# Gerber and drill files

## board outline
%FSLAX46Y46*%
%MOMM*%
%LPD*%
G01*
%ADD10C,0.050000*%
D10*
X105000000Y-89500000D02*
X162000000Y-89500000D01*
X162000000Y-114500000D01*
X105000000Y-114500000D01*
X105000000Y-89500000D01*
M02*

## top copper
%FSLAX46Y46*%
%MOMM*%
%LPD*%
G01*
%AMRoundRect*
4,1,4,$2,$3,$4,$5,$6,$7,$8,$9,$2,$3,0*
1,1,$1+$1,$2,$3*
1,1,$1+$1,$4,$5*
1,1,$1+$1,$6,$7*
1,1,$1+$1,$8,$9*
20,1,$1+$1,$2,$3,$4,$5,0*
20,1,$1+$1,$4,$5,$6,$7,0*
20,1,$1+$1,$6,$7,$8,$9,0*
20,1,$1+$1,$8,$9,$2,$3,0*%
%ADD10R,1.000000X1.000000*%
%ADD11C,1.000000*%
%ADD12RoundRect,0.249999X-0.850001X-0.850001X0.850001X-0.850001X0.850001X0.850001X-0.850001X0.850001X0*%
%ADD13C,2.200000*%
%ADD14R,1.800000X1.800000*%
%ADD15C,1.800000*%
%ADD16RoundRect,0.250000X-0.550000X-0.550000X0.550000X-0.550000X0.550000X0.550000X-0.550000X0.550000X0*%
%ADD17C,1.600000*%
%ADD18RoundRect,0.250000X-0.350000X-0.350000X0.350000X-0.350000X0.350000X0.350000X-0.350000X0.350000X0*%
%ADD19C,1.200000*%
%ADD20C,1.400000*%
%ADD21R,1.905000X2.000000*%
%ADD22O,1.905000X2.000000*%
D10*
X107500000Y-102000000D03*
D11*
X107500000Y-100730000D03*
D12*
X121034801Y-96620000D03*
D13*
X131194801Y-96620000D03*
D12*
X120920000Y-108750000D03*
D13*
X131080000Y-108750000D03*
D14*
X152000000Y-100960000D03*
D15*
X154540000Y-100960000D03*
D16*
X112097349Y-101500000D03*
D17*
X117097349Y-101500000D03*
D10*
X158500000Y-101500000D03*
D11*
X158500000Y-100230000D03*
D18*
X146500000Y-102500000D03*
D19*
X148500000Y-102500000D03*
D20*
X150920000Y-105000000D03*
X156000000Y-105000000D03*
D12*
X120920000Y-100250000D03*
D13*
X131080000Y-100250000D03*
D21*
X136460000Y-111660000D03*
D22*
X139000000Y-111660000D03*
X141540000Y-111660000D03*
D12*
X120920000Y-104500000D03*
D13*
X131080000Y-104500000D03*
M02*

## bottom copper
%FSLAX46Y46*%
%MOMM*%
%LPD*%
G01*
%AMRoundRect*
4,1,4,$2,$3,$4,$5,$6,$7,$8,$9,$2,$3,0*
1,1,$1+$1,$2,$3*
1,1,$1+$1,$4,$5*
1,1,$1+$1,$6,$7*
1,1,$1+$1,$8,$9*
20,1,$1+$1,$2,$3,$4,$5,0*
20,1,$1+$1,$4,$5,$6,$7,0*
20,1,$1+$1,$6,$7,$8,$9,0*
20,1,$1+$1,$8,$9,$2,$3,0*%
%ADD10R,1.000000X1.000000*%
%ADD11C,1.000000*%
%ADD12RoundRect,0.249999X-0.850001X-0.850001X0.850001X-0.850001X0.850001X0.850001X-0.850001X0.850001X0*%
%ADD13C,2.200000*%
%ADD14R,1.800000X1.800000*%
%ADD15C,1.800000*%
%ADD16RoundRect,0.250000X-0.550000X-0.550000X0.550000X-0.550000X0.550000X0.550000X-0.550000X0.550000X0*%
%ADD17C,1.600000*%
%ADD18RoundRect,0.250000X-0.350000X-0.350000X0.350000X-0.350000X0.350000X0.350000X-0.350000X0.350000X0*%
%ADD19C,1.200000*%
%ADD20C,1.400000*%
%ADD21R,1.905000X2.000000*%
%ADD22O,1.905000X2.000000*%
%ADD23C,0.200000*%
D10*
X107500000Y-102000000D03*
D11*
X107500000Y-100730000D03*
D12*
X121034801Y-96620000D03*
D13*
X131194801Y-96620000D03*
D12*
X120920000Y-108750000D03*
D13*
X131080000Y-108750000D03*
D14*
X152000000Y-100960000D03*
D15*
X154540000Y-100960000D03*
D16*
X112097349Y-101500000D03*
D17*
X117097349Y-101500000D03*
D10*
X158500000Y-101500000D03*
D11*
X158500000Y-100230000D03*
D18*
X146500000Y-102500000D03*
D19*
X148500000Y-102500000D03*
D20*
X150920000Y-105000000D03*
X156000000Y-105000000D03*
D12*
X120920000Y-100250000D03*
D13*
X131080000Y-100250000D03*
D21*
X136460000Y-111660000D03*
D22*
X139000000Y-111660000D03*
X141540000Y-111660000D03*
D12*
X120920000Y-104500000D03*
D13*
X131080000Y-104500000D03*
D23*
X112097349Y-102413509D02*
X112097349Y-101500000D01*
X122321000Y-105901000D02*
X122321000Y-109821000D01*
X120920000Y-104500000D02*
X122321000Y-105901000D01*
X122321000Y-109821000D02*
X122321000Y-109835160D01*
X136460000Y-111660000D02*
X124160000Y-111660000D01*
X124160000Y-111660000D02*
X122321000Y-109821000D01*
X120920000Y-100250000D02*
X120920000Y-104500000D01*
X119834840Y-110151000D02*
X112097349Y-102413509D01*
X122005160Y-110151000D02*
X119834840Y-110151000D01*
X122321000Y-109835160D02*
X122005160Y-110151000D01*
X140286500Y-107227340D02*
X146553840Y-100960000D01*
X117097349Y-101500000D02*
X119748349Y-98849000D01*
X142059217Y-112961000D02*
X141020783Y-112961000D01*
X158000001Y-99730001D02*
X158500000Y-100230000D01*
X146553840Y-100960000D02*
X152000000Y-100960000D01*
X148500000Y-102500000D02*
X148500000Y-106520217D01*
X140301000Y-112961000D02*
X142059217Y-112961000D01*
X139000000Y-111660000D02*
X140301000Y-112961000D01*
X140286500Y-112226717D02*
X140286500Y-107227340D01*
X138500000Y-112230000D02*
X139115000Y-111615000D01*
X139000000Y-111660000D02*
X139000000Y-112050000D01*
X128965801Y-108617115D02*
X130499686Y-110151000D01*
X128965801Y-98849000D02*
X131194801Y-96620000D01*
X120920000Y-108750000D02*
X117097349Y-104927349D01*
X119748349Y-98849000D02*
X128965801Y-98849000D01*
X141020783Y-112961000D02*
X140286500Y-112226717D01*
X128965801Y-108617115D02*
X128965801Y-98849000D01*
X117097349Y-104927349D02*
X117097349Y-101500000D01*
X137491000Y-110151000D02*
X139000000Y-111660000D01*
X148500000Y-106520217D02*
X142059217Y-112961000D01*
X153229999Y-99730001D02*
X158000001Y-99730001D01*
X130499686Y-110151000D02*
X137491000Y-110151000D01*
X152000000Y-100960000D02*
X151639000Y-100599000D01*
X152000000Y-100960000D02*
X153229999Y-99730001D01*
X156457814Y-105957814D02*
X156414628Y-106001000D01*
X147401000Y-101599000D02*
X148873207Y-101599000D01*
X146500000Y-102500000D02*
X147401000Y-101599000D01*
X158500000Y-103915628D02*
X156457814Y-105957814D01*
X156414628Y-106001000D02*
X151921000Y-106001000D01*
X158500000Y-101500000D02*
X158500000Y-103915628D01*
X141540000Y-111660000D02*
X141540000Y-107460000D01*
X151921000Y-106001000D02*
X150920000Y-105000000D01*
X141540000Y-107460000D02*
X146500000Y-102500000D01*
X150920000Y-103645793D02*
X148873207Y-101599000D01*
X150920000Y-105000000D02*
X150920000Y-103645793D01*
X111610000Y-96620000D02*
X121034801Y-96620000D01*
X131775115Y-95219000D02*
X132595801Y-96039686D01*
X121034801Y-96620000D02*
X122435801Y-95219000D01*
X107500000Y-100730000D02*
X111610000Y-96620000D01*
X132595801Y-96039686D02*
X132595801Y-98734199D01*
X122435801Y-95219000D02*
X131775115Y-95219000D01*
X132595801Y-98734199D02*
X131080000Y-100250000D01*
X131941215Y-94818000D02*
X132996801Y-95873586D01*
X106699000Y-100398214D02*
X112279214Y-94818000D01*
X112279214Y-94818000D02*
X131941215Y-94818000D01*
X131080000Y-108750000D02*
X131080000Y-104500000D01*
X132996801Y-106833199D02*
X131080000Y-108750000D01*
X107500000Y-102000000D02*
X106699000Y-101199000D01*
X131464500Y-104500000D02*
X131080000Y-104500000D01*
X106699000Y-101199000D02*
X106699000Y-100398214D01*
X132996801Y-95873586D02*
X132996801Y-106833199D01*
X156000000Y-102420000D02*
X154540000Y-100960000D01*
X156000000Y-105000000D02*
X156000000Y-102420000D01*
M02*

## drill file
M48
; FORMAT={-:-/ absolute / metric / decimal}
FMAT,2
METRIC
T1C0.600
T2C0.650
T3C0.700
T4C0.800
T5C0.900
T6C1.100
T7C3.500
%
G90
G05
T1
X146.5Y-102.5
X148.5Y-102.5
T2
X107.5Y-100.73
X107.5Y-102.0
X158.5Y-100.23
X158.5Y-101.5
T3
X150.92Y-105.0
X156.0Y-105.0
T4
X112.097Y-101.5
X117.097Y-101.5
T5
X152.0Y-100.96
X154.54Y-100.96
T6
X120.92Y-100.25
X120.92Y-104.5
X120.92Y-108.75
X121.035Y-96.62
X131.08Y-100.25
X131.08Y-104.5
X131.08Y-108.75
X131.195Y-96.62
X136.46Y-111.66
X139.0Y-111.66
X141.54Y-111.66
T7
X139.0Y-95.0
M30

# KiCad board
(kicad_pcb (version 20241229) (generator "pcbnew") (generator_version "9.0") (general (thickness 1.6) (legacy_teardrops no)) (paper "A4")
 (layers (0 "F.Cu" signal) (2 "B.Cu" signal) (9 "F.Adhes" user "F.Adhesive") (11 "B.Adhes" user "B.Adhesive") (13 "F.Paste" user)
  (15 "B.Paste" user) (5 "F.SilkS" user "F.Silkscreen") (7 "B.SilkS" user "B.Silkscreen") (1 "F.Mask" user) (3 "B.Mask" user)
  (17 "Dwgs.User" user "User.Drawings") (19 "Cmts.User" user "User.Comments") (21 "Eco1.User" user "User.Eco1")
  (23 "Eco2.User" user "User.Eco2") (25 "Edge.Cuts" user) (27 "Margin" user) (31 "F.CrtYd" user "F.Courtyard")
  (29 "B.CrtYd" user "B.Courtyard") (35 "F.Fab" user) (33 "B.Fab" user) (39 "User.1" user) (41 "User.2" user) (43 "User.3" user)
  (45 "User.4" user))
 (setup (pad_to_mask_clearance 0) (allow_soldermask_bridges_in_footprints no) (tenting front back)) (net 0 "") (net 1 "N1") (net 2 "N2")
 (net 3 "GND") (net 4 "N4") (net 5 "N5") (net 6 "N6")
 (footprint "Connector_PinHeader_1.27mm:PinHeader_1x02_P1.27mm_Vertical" (layer "F.Cu") (at 107.5 102 180)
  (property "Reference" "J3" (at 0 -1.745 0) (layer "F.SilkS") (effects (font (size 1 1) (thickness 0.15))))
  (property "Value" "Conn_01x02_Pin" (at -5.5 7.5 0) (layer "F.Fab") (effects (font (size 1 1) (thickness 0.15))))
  (pad "1" thru_hole rect (at 0 0 180) (size 1 1) (drill 0.65) (layers "*.Cu" "*.Mask") (remove_unused_layers no) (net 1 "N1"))
  (pad "2" thru_hole circle (at 0 1.27 180) (size 1 1) (drill 0.65) (layers "*.Cu" "*.Mask") (remove_unused_layers no) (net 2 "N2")))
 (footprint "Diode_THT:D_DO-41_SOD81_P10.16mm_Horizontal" (layer "F.Cu") (at 121.034801 96.62)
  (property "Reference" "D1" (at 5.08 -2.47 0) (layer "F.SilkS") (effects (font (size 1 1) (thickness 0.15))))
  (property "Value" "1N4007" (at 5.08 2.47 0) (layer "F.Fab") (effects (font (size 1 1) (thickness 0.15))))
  (pad "1" thru_hole roundrect (at 0 0) (size 2.2 2.2) (drill 1.1) (layers "*.Cu" "*.Mask") (remove_unused_layers no)
   (roundrect_rratio 0.113636) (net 2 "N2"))
  (pad "2" thru_hole circle (at 10.16 0) (size 2.2 2.2) (drill 1.1) (layers "*.Cu" "*.Mask") (remove_unused_layers no) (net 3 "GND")))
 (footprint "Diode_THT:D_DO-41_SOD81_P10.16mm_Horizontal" (layer "F.Cu") (at 120.92 108.75)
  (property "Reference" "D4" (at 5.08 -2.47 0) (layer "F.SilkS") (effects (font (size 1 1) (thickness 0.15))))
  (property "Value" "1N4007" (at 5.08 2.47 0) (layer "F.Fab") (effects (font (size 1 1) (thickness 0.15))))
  (pad "1" thru_hole roundrect (at 0 0) (size 2.2 2.2) (drill 1.1) (layers "*.Cu" "*.Mask") (remove_unused_layers no)
   (roundrect_rratio 0.113636) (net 3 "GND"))
  (pad "2" thru_hole circle (at 10.16 0) (size 2.2 2.2) (drill 1.1) (layers "*.Cu" "*.Mask") (remove_unused_layers no) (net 1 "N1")))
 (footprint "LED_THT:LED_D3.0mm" (layer "F.Cu") (at 152 100.96)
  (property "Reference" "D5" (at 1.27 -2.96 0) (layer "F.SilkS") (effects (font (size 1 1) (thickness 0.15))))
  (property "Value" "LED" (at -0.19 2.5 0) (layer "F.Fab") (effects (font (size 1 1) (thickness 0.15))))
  (pad "1" thru_hole rect (at 0 0) (size 1.8 1.8) (drill 0.9) (layers "*.Cu" "*.Mask") (remove_unused_layers no) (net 3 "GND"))
  (pad "2" thru_hole circle (at 2.54 0) (size 1.8 1.8) (drill 0.9) (layers "*.Cu" "*.Mask") (remove_unused_layers no) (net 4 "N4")))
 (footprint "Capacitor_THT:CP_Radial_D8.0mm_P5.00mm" (layer "F.Cu") (at 112.097349 101.5)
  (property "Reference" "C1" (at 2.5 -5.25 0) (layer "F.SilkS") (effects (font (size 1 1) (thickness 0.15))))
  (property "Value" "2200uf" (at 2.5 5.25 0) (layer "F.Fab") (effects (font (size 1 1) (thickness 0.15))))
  (pad "1" thru_hole roundrect (at 0 0) (size 1.6 1.6) (drill 0.8) (layers "*.Cu" "*.Mask") (remove_unused_layers no)
   (roundrect_rratio 0.15625) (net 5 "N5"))
  (pad "2" thru_hole circle (at 5 0) (size 1.6 1.6) (drill 0.8) (layers "*.Cu" "*.Mask") (remove_unused_layers no) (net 3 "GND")))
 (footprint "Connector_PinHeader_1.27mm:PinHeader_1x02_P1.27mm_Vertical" (layer "F.Cu") (at 158.5 101.5 180)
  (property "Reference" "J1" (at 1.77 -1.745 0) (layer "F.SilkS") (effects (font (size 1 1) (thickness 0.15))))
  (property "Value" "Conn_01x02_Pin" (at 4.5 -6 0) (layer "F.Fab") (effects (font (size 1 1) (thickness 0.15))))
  (pad "1" thru_hole rect (at 0 0 180) (size 1 1) (drill 0.65) (layers "*.Cu" "*.Mask") (remove_unused_layers no) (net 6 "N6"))
  (pad "2" thru_hole circle (at 0 1.27 180) (size 1 1) (drill 0.65) (layers "*.Cu" "*.Mask") (remove_unused_layers no) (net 3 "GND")))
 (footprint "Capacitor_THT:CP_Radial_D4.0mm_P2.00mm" (layer "F.Cu") (at 146.5 102.5)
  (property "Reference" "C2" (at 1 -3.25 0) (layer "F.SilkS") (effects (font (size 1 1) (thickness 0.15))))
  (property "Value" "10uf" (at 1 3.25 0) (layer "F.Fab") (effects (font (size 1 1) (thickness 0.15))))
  (pad "1" thru_hole roundrect (at 0 0) (size 1.2 1.2) (drill 0.6) (layers "*.Cu" "*.Mask") (remove_unused_layers no)
   (roundrect_rratio 0.208333) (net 6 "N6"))
  (pad "2" thru_hole circle (at 2 0) (size 1.2 1.2) (drill 0.6) (layers "*.Cu" "*.Mask") (remove_unused_layers no) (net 3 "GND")))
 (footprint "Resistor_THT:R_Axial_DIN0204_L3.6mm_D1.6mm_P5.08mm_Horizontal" (layer "F.Cu") (at 150.92 105)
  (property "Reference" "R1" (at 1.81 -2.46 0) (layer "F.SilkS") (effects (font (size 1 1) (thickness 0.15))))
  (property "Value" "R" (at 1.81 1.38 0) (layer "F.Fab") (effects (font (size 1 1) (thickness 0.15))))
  (pad "1" thru_hole circle (at 0 0) (size 1.4 1.4) (drill 0.7) (layers "*.Cu" "*.Mask") (remove_unused_layers no) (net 6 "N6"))
  (pad "2" thru_hole circle (at 5.08 0) (size 1.4 1.4) (drill 0.7) (layers "*.Cu" "*.Mask") (remove_unused_layers no) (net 4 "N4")))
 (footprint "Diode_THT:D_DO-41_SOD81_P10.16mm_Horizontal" (layer "F.Cu") (at 120.92 100.25)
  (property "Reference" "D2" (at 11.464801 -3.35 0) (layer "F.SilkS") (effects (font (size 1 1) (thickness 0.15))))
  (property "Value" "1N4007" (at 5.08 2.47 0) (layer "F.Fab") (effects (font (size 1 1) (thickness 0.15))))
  (pad "1" thru_hole roundrect (at 0 0) (size 2.2 2.2) (drill 1.1) (layers "*.Cu" "*.Mask") (remove_unused_layers no)
   (roundrect_rratio 0.113636) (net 5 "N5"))
  (pad "2" thru_hole circle (at 10.16 0) (size 2.2 2.2) (drill 1.1) (layers "*.Cu" "*.Mask") (remove_unused_layers no) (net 2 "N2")))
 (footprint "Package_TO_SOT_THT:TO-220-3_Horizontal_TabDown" (layer "F.Cu") (at 136.46 111.66)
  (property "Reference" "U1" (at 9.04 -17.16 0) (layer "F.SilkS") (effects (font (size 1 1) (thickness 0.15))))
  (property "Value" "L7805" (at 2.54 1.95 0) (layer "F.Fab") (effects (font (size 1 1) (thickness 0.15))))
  (pad "" np_thru_hole circle (at 2.54 -16.66) (size 3.5 3.5) (drill 3.5) (layers "*.Cu" "*.Mask"))
  (pad "1" thru_hole rect (at 0 0) (size 1.905 2) (drill 1.1) (layers "*.Cu" "*.Mask") (remove_unused_layers no) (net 5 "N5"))
  (pad "2" thru_hole oval (at 2.54 0) (size 1.905 2) (drill 1.1) (layers "*.Cu" "*.Mask") (remove_unused_layers no) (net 3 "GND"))
  (pad "3" thru_hole oval (at 5.08 0) (size 1.905 2) (drill 1.1) (layers "*.Cu" "*.Mask") (remove_unused_layers no) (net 6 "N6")))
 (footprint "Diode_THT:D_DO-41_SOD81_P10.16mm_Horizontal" (layer "F.Cu") (at 120.92 104.5)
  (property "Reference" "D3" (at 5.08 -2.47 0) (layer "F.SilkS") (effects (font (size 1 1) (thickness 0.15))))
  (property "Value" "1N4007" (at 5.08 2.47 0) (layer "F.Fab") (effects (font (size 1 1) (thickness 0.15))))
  (pad "1" thru_hole roundrect (at 0 0) (size 2.2 2.2) (drill 1.1) (layers "*.Cu" "*.Mask") (remove_unused_layers no)
   (roundrect_rratio 0.113636) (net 5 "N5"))
  (pad "2" thru_hole circle (at 10.16 0) (size 2.2 2.2) (drill 1.1) (layers "*.Cu" "*.Mask") (remove_unused_layers no) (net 1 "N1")))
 (gr_rect (start 105 89.5) (end 162 114.5) (stroke (width 0.05) (type default)) (fill no) (layer "Edge.Cuts"))
 (segment (start 112.097349 102.413509) (end 112.097349 101.5) (width 0.2) (layer "B.Cu") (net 5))
 (segment (start 122.321 105.901) (end 122.321 109.821) (width 0.2) (layer "B.Cu") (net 5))
 (segment (start 120.92 104.5) (end 122.321 105.901) (width 0.2) (layer "B.Cu") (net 5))
 (segment (start 122.321 109.821) (end 122.321 109.83516) (width 0.2) (layer "B.Cu") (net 5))
 (segment (start 136.46 111.66) (end 124.16 111.66) (width 0.2) (layer "B.Cu") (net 5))
 (segment (start 124.16 111.66) (end 122.321 109.821) (width 0.2) (layer "B.Cu") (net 5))
 (segment (start 120.92 100.25) (end 120.92 104.5) (width 0.2) (layer "B.Cu") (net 5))
 (segment (start 119.83484 110.151) (end 112.097349 102.413509) (width 0.2) (layer "B.Cu") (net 5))
 (segment (start 122.00516 110.151) (end 119.83484 110.151) (width 0.2) (layer "B.Cu") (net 5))
 (segment (start 122.321 109.83516) (end 122.00516 110.151) (width 0.2) (layer "B.Cu") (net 5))
 (segment (start 140.2865 107.22734) (end 146.55384 100.96) (width 0.2) (layer "B.Cu") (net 3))
 (segment (start 117.097349 101.5) (end 119.748349 98.849) (width 0.2) (layer "B.Cu") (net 3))
 (segment (start 142.059217 112.961) (end 141.020783 112.961) (width 0.2) (layer "B.Cu") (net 3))
 (segment (start 158.000001 99.730001) (end 158.5 100.23) (width 0.2) (layer "B.Cu") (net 3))
 (segment (start 146.55384 100.96) (end 152 100.96) (width 0.2) (layer "B.Cu") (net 3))
 (segment (start 148.5 102.5) (end 148.5 106.520217) (width 0.2) (layer "B.Cu") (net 3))
 (segment (start 140.301 112.961) (end 142.059217 112.961) (width 0.2) (layer "B.Cu") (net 3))
 (segment (start 139 111.66) (end 140.301 112.961) (width 0.2) (layer "B.Cu") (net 3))
 (segment (start 140.2865 112.226717) (end 140.2865 107.22734) (width 0.2) (layer "B.Cu") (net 3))
 (segment (start 138.5 112.23) (end 139.115 111.615) (width 0.2) (layer "B.Cu") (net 3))
 (segment (start 139 111.66) (end 139 112.05) (width 0.2) (layer "B.Cu") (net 3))
 (segment (start 128.965801 108.617115) (end 130.499686 110.151) (width 0.2) (layer "B.Cu") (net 3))
 (segment (start 128.965801 98.849) (end 131.194801 96.62) (width 0.2) (layer "B.Cu") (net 3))
 (segment (start 120.92 108.75) (end 117.097349 104.927349) (width 0.2) (layer "B.Cu") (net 3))
 (segment (start 119.748349 98.849) (end 128.965801 98.849) (width 0.2) (layer "B.Cu") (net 3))
 (segment (start 141.020783 112.961) (end 140.2865 112.226717) (width 0.2) (layer "B.Cu") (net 3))
 (segment (start 128.965801 108.617115) (end 128.965801 98.849) (width 0.2) (layer "B.Cu") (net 3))
 (segment (start 117.097349 104.927349) (end 117.097349 101.5) (width 0.2) (layer "B.Cu") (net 3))
 (segment (start 137.491 110.151) (end 139 111.66) (width 0.2) (layer "B.Cu") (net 3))
 (segment (start 148.5 106.520217) (end 142.059217 112.961) (width 0.2) (layer "B.Cu") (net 3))
 (segment (start 153.229999 99.730001) (end 158.000001 99.730001) (width 0.2) (layer "B.Cu") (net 3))
 (segment (start 130.499686 110.151) (end 137.491 110.151) (width 0.2) (layer "B.Cu") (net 3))
 (segment (start 152 100.96) (end 151.639 100.599) (width 0.2) (layer "B.Cu") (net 3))
 (segment (start 152 100.96) (end 153.229999 99.730001) (width 0.2) (layer "B.Cu") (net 3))
 (segment (start 156.457814 105.957814) (end 156.414628 106.001) (width 0.2) (layer "B.Cu") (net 6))
 (segment (start 147.401 101.599) (end 148.873207 101.599) (width 0.2) (layer "B.Cu") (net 6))
 (segment (start 146.5 102.5) (end 147.401 101.599) (width 0.2) (layer "B.Cu") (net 6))
 (segment (start 158.5 103.915628) (end 156.457814 105.957814) (width 0.2) (layer "B.Cu") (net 6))
 (segment (start 156.414628 106.001) (end 151.921 106.001) (width 0.2) (layer "B.Cu") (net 6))
 (segment (start 158.5 101.5) (end 158.5 103.915628) (width 0.2) (layer "B.Cu") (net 6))
 (segment (start 141.54 111.66) (end 141.54 107.46) (width 0.2) (layer "B.Cu") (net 6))
 (segment (start 151.921 106.001) (end 150.92 105) (width 0.2) (layer "B.Cu") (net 6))
 (segment (start 141.54 107.46) (end 146.5 102.5) (width 0.2) (layer "B.Cu") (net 6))
 (segment (start 150.92 103.645793) (end 148.873207 101.599) (width 0.2) (layer "B.Cu") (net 6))
 (segment (start 150.92 105) (end 150.92 103.645793) (width 0.2) (layer "B.Cu") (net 6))
 (segment (start 111.61 96.62) (end 121.034801 96.62) (width 0.2) (layer "B.Cu") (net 2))
 (segment (start 131.775115 95.219) (end 132.595801 96.039686) (width 0.2) (layer "B.Cu") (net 2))
 (segment (start 121.034801 96.62) (end 122.435801 95.219) (width 0.2) (layer "B.Cu") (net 2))
 (segment (start 107.5 100.73) (end 111.61 96.62) (width 0.2) (layer "B.Cu") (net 2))
 (segment (start 132.595801 96.039686) (end 132.595801 98.734199) (width 0.2) (layer "B.Cu") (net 2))
 (segment (start 122.435801 95.219) (end 131.775115 95.219) (width 0.2) (layer "B.Cu") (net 2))
 (segment (start 132.595801 98.734199) (end 131.08 100.25) (width 0.2) (layer "B.Cu") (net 2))
 (segment (start 131.941215 94.818) (end 132.996801 95.873586) (width 0.2) (layer "B.Cu") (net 1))
 (segment (start 106.699 100.398214) (end 112.279214 94.818) (width 0.2) (layer "B.Cu") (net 1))
 (segment (start 112.279214 94.818) (end 131.941215 94.818) (width 0.2) (layer "B.Cu") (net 1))
 (segment (start 131.08 108.75) (end 131.08 104.5) (width 0.2) (layer "B.Cu") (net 1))
 (segment (start 132.996801 106.833199) (end 131.08 108.75) (width 0.2) (layer "B.Cu") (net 1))
 (segment (start 107.5 102) (end 106.699 101.199) (width 0.2) (layer "B.Cu") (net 1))
 (segment (start 131.4645 104.5) (end 131.08 104.5) (width 0.2) (layer "B.Cu") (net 1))
 (segment (start 106.699 101.199) (end 106.699 100.398214) (width 0.2) (layer "B.Cu") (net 1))
 (segment (start 132.996801 95.873586) (end 132.996801 106.833199) (width 0.2) (layer "B.Cu") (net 1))
 (segment (start 156 102.42) (end 154.54 100.96) (width 0.2) (layer "B.Cu") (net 4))
 (segment (start 156 105) (end 156 102.42) (width 0.2) (layer "B.Cu") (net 4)))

